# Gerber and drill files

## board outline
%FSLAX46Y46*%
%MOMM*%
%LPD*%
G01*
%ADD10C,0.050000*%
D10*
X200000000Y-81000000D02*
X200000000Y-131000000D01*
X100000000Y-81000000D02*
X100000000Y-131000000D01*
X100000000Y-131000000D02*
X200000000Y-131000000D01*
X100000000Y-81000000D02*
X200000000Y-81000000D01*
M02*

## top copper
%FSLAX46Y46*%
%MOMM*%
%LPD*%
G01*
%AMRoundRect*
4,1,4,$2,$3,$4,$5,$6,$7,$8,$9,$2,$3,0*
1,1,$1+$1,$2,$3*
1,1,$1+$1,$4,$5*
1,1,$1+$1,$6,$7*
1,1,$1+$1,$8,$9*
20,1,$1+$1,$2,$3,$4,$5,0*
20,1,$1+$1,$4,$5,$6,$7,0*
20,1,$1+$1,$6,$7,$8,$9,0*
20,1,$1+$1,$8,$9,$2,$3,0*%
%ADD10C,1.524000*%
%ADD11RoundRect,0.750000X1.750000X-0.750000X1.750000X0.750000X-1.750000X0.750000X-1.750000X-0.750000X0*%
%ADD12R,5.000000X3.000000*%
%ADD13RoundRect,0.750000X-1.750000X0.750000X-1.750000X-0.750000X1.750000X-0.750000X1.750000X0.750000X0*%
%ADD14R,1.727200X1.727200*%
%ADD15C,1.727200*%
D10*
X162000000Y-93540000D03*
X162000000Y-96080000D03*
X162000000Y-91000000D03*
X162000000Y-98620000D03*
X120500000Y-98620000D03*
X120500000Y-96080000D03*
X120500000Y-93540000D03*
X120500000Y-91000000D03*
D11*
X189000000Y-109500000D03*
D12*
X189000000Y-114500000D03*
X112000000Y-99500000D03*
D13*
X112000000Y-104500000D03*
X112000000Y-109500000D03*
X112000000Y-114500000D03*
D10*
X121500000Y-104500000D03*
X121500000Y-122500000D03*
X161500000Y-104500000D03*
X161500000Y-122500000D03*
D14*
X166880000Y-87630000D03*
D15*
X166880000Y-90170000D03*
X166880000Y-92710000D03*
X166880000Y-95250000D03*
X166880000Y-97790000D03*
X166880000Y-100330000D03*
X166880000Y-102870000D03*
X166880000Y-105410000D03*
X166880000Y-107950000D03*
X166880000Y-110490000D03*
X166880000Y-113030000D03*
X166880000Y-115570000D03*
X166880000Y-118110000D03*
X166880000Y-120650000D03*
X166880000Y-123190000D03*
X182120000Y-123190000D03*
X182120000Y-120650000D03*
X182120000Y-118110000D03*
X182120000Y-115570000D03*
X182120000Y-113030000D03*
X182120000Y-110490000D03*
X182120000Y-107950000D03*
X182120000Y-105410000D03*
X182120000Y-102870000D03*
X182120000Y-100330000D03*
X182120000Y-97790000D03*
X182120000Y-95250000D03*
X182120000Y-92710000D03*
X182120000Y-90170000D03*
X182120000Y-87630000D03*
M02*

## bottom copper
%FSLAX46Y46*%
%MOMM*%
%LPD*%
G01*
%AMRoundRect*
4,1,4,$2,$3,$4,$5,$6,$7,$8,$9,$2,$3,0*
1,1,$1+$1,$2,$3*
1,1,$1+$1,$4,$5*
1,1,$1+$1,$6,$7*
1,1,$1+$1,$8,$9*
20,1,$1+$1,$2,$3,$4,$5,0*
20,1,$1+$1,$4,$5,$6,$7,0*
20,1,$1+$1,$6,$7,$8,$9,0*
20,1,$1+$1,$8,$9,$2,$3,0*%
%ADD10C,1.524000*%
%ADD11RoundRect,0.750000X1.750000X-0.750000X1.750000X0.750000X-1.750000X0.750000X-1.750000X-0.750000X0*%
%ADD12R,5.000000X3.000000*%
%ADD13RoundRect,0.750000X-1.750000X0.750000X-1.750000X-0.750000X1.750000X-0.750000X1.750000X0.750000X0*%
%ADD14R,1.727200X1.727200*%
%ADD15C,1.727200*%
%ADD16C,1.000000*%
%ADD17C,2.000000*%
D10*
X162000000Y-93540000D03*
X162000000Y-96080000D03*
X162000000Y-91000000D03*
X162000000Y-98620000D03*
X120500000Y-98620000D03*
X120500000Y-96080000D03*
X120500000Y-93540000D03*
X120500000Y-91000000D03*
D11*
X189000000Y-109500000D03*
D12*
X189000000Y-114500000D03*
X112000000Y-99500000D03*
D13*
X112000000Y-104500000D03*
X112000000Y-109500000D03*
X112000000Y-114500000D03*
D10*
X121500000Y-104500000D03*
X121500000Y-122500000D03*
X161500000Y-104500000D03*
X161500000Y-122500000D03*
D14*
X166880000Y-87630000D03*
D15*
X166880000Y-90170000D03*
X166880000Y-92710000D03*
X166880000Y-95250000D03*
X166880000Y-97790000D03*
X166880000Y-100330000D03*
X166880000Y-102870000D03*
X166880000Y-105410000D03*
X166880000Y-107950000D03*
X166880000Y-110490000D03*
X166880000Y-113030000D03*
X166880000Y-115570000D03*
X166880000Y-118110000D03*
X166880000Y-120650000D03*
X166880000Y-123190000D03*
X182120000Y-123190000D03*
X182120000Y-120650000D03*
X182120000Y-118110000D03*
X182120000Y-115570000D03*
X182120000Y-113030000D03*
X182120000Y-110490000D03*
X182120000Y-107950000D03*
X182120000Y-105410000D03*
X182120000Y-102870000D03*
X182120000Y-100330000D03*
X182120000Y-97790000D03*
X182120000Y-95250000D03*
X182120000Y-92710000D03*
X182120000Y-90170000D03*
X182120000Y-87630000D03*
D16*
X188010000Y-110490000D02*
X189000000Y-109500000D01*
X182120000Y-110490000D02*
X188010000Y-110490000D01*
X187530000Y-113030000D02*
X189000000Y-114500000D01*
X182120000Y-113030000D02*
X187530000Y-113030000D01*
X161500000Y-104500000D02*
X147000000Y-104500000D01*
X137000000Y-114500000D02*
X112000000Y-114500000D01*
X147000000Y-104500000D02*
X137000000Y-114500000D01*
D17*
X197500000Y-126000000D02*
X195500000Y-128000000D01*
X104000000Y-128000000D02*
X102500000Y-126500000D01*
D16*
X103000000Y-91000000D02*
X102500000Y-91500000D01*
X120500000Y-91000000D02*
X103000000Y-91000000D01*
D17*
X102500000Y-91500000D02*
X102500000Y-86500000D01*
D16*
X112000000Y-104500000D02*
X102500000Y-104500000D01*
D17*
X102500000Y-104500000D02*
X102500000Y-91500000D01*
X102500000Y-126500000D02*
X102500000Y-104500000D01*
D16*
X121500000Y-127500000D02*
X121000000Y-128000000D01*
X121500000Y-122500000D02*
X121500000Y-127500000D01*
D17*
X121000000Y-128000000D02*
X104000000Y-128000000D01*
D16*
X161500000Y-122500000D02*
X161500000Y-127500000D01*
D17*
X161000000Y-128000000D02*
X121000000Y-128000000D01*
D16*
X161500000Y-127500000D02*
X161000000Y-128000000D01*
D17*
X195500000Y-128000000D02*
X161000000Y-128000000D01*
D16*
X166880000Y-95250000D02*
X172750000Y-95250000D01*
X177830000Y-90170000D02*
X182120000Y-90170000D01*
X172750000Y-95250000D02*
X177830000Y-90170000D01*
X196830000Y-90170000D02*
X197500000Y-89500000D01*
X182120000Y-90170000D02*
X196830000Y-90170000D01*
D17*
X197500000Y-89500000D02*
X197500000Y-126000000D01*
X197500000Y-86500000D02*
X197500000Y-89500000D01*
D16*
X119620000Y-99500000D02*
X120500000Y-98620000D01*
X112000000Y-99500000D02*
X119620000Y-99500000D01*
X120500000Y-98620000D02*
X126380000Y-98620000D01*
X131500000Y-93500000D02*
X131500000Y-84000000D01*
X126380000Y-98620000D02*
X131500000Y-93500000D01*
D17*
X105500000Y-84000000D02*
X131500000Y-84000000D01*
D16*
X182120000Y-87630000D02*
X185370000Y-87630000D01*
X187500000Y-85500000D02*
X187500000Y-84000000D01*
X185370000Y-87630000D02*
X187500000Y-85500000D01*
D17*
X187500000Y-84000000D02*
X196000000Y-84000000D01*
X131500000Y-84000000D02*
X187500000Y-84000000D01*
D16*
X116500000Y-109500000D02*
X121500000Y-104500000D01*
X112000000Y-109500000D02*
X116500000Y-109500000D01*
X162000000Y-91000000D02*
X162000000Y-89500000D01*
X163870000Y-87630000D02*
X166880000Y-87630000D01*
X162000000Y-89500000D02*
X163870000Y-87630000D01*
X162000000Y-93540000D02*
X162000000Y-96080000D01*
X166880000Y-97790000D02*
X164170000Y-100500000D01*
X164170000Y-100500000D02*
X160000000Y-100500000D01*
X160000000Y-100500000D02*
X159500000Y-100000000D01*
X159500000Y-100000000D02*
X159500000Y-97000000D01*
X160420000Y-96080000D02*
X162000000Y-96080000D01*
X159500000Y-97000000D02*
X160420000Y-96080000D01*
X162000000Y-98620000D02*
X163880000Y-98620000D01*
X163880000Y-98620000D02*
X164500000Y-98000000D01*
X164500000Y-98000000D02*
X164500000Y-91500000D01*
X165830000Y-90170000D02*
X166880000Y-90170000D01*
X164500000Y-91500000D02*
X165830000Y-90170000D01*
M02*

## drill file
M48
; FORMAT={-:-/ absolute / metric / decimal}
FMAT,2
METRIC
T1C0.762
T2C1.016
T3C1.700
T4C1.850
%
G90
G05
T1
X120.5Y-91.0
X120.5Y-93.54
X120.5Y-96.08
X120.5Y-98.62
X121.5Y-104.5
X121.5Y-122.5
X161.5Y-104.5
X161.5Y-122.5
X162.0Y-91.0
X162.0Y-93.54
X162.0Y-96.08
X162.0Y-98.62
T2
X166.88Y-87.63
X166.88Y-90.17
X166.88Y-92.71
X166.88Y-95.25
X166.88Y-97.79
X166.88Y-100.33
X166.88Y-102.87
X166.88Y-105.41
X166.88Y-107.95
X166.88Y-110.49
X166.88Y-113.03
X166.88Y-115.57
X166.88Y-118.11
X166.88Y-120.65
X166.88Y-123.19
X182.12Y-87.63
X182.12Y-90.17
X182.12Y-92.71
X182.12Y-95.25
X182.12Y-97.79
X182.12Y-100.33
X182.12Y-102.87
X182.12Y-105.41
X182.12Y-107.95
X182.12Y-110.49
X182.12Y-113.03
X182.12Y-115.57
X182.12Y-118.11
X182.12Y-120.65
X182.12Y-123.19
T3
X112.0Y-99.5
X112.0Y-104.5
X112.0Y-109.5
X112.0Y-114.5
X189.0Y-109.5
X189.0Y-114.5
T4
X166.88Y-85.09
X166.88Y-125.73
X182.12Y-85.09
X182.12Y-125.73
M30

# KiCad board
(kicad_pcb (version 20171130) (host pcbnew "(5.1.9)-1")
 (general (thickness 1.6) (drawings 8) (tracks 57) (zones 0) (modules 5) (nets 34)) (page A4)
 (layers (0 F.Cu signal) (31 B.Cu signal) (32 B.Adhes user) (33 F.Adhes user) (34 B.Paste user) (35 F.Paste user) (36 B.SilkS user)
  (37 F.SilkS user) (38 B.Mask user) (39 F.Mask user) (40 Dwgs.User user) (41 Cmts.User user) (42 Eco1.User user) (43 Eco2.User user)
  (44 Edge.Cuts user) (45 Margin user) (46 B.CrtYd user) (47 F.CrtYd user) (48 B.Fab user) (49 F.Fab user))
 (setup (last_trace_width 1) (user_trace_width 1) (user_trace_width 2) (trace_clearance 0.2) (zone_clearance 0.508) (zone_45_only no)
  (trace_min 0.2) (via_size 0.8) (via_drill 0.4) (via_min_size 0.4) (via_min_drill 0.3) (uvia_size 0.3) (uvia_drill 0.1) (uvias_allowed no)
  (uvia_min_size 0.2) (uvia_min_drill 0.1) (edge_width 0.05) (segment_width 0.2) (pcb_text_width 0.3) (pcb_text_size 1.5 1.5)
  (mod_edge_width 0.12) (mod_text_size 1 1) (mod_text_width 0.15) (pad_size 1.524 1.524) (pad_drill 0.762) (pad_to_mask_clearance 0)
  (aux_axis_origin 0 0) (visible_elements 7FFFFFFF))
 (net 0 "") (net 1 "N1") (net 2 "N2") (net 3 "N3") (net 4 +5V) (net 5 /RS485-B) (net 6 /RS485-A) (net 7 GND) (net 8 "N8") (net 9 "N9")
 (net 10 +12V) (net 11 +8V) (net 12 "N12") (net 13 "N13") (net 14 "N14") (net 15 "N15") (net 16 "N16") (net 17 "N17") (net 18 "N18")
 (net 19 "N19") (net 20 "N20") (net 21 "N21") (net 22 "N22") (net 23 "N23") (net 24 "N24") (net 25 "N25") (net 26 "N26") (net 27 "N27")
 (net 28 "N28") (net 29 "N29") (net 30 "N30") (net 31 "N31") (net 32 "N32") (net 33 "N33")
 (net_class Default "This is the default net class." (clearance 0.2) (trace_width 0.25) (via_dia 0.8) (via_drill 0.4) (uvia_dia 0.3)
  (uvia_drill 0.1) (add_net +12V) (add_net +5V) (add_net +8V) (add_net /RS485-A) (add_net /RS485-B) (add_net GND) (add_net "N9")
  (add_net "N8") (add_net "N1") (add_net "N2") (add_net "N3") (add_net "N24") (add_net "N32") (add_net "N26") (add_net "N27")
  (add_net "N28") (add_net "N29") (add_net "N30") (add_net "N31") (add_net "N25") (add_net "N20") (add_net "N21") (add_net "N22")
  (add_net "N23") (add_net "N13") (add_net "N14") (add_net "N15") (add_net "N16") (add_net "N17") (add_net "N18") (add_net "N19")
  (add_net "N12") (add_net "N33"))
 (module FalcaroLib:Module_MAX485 (layer F.Cu) (at 120.5 91)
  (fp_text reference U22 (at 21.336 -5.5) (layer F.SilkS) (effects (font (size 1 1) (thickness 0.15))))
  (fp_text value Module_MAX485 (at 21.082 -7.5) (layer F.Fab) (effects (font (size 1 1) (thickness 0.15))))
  (pad DE thru_hole circle (at 41.5 2.54) (size 1.524 1.524) (drill 0.762) (layers *.Cu *.Mask) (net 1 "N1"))
  (pad RE thru_hole circle (at 41.5 5.08) (size 1.524 1.524) (drill 0.762) (layers *.Cu *.Mask) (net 1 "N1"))
  (pad DI thru_hole circle (at 41.5 0) (size 1.524 1.524) (drill 0.762) (layers *.Cu *.Mask) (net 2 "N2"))
  (pad RO thru_hole circle (at 41.5 7.62) (size 1.524 1.524) (drill 0.762) (layers *.Cu *.Mask) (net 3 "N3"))
  (pad VCC thru_hole circle (at 0 7.62) (size 1.524 1.524) (drill 0.762) (layers *.Cu *.Mask) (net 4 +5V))
  (pad B thru_hole circle (at 0 5.08) (size 1.524 1.524) (drill 0.762) (layers *.Cu *.Mask) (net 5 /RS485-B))
  (pad A thru_hole circle (at 0 2.54) (size 1.524 1.524) (drill 0.762) (layers *.Cu *.Mask) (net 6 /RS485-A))
  (pad GND thru_hole circle (at 0 0) (size 1.524 1.524) (drill 0.762) (layers *.Cu *.Mask) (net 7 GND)))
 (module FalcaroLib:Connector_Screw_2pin (layer F.Cu) (at 184.5 118 90)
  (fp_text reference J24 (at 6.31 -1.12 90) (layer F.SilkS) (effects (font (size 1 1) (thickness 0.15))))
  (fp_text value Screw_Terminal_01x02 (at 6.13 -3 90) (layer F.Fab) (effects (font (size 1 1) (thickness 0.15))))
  (pad 2 thru_hole roundrect (at 8.5 4.5 90) (size 3 5) (drill 1.7) (layers *.Cu *.Mask) (roundrect_rratio 0.25) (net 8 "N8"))
  (pad 1 thru_hole rect (at 3.5 4.5 90) (size 3 5) (drill 1.7) (layers *.Cu *.Mask) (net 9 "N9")))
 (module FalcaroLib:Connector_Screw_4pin (layer F.Cu) (at 116.5 96 270)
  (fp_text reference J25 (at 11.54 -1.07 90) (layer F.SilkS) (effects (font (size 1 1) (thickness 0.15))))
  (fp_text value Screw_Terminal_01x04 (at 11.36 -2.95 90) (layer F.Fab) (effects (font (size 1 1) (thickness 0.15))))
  (pad 1 thru_hole rect (at 3.5 4.5 270) (size 3 5) (drill 1.7) (layers *.Cu *.Mask) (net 4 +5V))
  (pad 2 thru_hole roundrect (at 8.5 4.5 270) (size 3 5) (drill 1.7) (layers *.Cu *.Mask) (roundrect_rratio 0.25) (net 7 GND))
  (pad 3 thru_hole roundrect (at 13.5 4.5 270) (size 3 5) (drill 1.7) (layers *.Cu *.Mask) (roundrect_rratio 0.25) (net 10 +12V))
  (pad 4 thru_hole roundrect (at 18.5 4.5 270) (size 3 5) (drill 1.7) (layers *.Cu *.Mask) (roundrect_rratio 0.25) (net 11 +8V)))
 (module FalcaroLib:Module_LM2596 (layer F.Cu) (at 121.5 104.5)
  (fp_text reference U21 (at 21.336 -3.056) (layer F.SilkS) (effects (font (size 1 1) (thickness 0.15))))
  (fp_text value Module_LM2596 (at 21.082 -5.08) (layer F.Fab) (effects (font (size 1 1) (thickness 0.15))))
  (pad IN+ thru_hole circle (at 0 0) (size 1.524 1.524) (drill 0.762) (layers *.Cu *.Mask) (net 10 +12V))
  (pad IN- thru_hole circle (at 0 18) (size 1.524 1.524) (drill 0.762) (layers *.Cu *.Mask) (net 7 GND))
  (pad OUT+ thru_hole circle (at 40 0) (size 1.524 1.524) (drill 0.762) (layers *.Cu *.Mask) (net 11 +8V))
  (pad OUT- thru_hole circle (at 40 18) (size 1.524 1.524) (drill 0.762) (layers *.Cu *.Mask) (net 7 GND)))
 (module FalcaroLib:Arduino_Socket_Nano (layer F.Cu) (at 174.5 127)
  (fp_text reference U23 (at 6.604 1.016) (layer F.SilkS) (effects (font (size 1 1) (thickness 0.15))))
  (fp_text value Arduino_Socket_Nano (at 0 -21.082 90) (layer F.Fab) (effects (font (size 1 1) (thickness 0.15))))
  (pad "" np_thru_hole circle (at 7.62 -1.27) (size 1.85 1.85) (drill 1.85) (layers *.Cu *.Mask))
  (pad "" np_thru_hole circle (at -7.62 -1.27) (size 1.85 1.85) (drill 1.85) (layers *.Cu *.Mask))
  (pad "" np_thru_hole circle (at 7.62 -41.91) (size 1.85 1.85) (drill 1.85) (layers *.Cu *.Mask))
  (pad "" np_thru_hole circle (at -7.62 -41.91) (size 1.85 1.85) (drill 1.85) (layers *.Cu *.Mask))
  (pad D1 thru_hole rect (at -7.62 -39.37) (size 1.7272 1.7272) (drill 1.016) (layers *.Cu *.Mask) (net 2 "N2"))
  (pad D0 thru_hole circle (at -7.62 -36.83) (size 1.7272 1.7272) (drill 1.016) (layers *.Cu *.Mask) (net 3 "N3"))
  (pad RST1 thru_hole circle (at -7.62 -34.29) (size 1.7272 1.7272) (drill 1.016) (layers *.Cu *.Mask) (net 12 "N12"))
  (pad GND1 thru_hole circle (at -7.62 -31.75) (size 1.7272 1.7272) (drill 1.016) (layers *.Cu *.Mask) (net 7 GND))
  (pad D2 thru_hole circle (at -7.62 -29.21) (size 1.7272 1.7272) (drill 1.016) (layers *.Cu *.Mask) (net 1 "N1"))
  (pad D3 thru_hole circle (at -7.62 -26.67) (size 1.7272 1.7272) (drill 1.016) (layers *.Cu *.Mask) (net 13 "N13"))
  (pad D4 thru_hole circle (at -7.62 -24.13) (size 1.7272 1.7272) (drill 1.016) (layers *.Cu *.Mask) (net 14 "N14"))
  (pad D5 thru_hole circle (at -7.62 -21.59) (size 1.7272 1.7272) (drill 1.016) (layers *.Cu *.Mask) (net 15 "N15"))
  (pad D6 thru_hole circle (at -7.62 -19.05) (size 1.7272 1.7272) (drill 1.016) (layers *.Cu *.Mask) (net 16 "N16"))
  (pad D7 thru_hole circle (at -7.62 -16.51) (size 1.7272 1.7272) (drill 1.016) (layers *.Cu *.Mask) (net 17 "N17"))
  (pad D8 thru_hole circle (at -7.62 -13.97) (size 1.7272 1.7272) (drill 1.016) (layers *.Cu *.Mask) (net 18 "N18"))
  (pad D9 thru_hole circle (at -7.62 -11.43) (size 1.7272 1.7272) (drill 1.016) (layers *.Cu *.Mask) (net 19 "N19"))
  (pad D10 thru_hole circle (at -7.62 -8.89) (size 1.7272 1.7272) (drill 1.016) (layers *.Cu *.Mask) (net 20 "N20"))
  (pad D11 thru_hole circle (at -7.62 -6.35) (size 1.7272 1.7272) (drill 1.016) (layers *.Cu *.Mask) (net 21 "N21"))
  (pad D12 thru_hole circle (at -7.62 -3.81) (size 1.7272 1.7272) (drill 1.016) (layers *.Cu *.Mask) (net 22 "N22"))
  (pad D13 thru_hole circle (at 7.62 -3.81) (size 1.7272 1.7272) (drill 1.016) (layers *.Cu *.Mask) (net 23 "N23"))
  (pad 3V3 thru_hole circle (at 7.62 -6.35) (size 1.7272 1.7272) (drill 1.016) (layers *.Cu *.Mask) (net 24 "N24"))
  (pad AREF thru_hole circle (at 7.62 -8.89) (size 1.7272 1.7272) (drill 1.016) (layers *.Cu *.Mask) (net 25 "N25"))
  (pad A0 thru_hole circle (at 7.62 -11.43) (size 1.7272 1.7272) (drill 1.016) (layers *.Cu *.Mask) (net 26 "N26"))
  (pad A1 thru_hole circle (at 7.62 -13.97) (size 1.7272 1.7272) (drill 1.016) (layers *.Cu *.Mask) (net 9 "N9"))
  (pad A2 thru_hole circle (at 7.62 -16.51) (size 1.7272 1.7272) (drill 1.016) (layers *.Cu *.Mask) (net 8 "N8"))
  (pad A3 thru_hole circle (at 7.62 -19.05) (size 1.7272 1.7272) (drill 1.016) (layers *.Cu *.Mask) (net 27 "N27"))
  (pad A4 thru_hole circle (at 7.62 -21.59) (size 1.7272 1.7272) (drill 1.016) (layers *.Cu *.Mask) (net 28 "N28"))
  (pad A5 thru_hole circle (at 7.62 -24.13) (size 1.7272 1.7272) (drill 1.016) (layers *.Cu *.Mask) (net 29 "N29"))
  (pad A6 thru_hole circle (at 7.62 -26.67) (size 1.7272 1.7272) (drill 1.016) (layers *.Cu *.Mask) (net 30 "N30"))
  (pad A7 thru_hole circle (at 7.62 -29.21) (size 1.7272 1.7272) (drill 1.016) (layers *.Cu *.Mask) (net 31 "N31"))
  (pad 5V thru_hole circle (at 7.62 -31.75) (size 1.7272 1.7272) (drill 1.016) (layers *.Cu *.Mask) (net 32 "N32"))
  (pad RST2 thru_hole circle (at 7.62 -34.29) (size 1.7272 1.7272) (drill 1.016) (layers *.Cu *.Mask) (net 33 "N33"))
  (pad GND2 thru_hole circle (at 7.62 -36.83) (size 1.7272 1.7272) (drill 1.016) (layers *.Cu *.Mask) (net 7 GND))
  (pad VIN thru_hole circle (at 7.62 -39.37) (size 1.7272 1.7272) (drill 1.016) (layers *.Cu *.Mask) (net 4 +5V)))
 (gr_line (start 200 81) (end 200 131) (layer Edge.Cuts) (width 0.05))
 (gr_line (start 100 81) (end 100 131) (layer Edge.Cuts) (width 0.05))
 (gr_line (start 100 131) (end 200 131) (layer Edge.Cuts) (width 0.05))
 (gr_line (start 100 81) (end 200 81) (layer Edge.Cuts) (width 0.05))
 (segment (start 188.01 110.49) (end 189 109.5) (width 1) (layer B.Cu) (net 8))
 (segment (start 182.12 110.49) (end 188.01 110.49) (width 1) (layer B.Cu) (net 8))
 (segment (start 187.53 113.03) (end 189 114.5) (width 1) (layer B.Cu) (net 9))
 (segment (start 182.12 113.03) (end 187.53 113.03) (width 1) (layer B.Cu) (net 9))
 (segment (start 161.5 104.5) (end 147 104.5) (width 1) (layer B.Cu) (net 11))
 (segment (start 137 114.5) (end 112 114.5) (width 1) (layer B.Cu) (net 11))
 (segment (start 147 104.5) (end 137 114.5) (width 1) (layer B.Cu) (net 11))
 (segment (start 197.5 126) (end 195.5 128) (width 2) (layer B.Cu) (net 7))
 (segment (start 104 128) (end 102.5 126.5) (width 2) (layer B.Cu) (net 7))
 (segment (start 103 91) (end 102.5 91.5) (width 1) (layer B.Cu) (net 7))
 (segment (start 120.5 91) (end 103 91) (width 1) (layer B.Cu) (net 7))
 (segment (start 102.5 91.5) (end 102.5 86.5) (width 2) (layer B.Cu) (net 7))
 (segment (start 112 104.5) (end 102.5 104.5) (width 1) (layer B.Cu) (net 7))
 (segment (start 102.5 104.5) (end 102.5 91.5) (width 2) (layer B.Cu) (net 7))
 (segment (start 102.5 126.5) (end 102.5 104.5) (width 2) (layer B.Cu) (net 7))
 (segment (start 121.5 127.5) (end 121 128) (width 1) (layer B.Cu) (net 7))
 (segment (start 121.5 122.5) (end 121.5 127.5) (width 1) (layer B.Cu) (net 7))
 (segment (start 121 128) (end 104 128) (width 2) (layer B.Cu) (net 7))
 (segment (start 161.5 122.5) (end 161.5 127.5) (width 1) (layer B.Cu) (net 7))
 (segment (start 161 128) (end 121 128) (width 2) (layer B.Cu) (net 7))
 (segment (start 161.5 127.5) (end 161 128) (width 1) (layer B.Cu) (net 7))
 (segment (start 195.5 128) (end 161 128) (width 2) (layer B.Cu) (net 7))
 (segment (start 166.88 95.25) (end 172.75 95.25) (width 1) (layer B.Cu) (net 7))
 (segment (start 177.83 90.17) (end 182.12 90.17) (width 1) (layer B.Cu) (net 7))
 (segment (start 172.75 95.25) (end 177.83 90.17) (width 1) (layer B.Cu) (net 7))
 (segment (start 196.83 90.17) (end 197.5 89.5) (width 1) (layer B.Cu) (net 7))
 (segment (start 182.12 90.17) (end 196.83 90.17) (width 1) (layer B.Cu) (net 7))
 (segment (start 197.5 89.5) (end 197.5 126) (width 2) (layer B.Cu) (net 7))
 (segment (start 197.5 86.5) (end 197.5 89.5) (width 2) (layer B.Cu) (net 7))
 (segment (start 119.62 99.5) (end 120.5 98.62) (width 1) (layer B.Cu) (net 4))
 (segment (start 112 99.5) (end 119.62 99.5) (width 1) (layer B.Cu) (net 4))
 (segment (start 120.5 98.62) (end 126.38 98.62) (width 1) (layer B.Cu) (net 4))
 (segment (start 131.5 93.5) (end 131.5 84) (width 1) (layer B.Cu) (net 4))
 (segment (start 126.38 98.62) (end 131.5 93.5) (width 1) (layer B.Cu) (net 4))
 (segment (start 105.5 84) (end 131.5 84) (width 2) (layer B.Cu) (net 4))
 (segment (start 182.12 87.63) (end 185.37 87.63) (width 1) (layer B.Cu) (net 4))
 (segment (start 187.5 85.5) (end 187.5 84) (width 1) (layer B.Cu) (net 4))
 (segment (start 185.37 87.63) (end 187.5 85.5) (width 1) (layer B.Cu) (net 4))
 (segment (start 187.5 84) (end 196 84) (width 2) (layer B.Cu) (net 4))
 (segment (start 131.5 84) (end 187.5 84) (width 2) (layer B.Cu) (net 4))
 (segment (start 116.5 109.5) (end 121.5 104.5) (width 1) (layer B.Cu) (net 10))
 (segment (start 112 109.5) (end 116.5 109.5) (width 1) (layer B.Cu) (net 10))
 (segment (start 162 91) (end 162 89.5) (width 1) (layer B.Cu) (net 2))
 (segment (start 163.87 87.63) (end 166.88 87.63) (width 1) (layer B.Cu) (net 2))
 (segment (start 162 89.5) (end 163.87 87.63) (width 1) (layer B.Cu) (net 2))
 (segment (start 162 93.54) (end 162 96.08) (width 1) (layer B.Cu) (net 1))
 (segment (start 166.88 97.79) (end 164.17 100.5) (width 1) (layer B.Cu) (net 1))
 (segment (start 164.17 100.5) (end 160 100.5) (width 1) (layer B.Cu) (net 1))
 (segment (start 160 100.5) (end 159.5 100) (width 1) (layer B.Cu) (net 1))
 (segment (start 159.5 100) (end 159.5 97) (width 1) (layer B.Cu) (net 1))
 (segment (start 160.42 96.08) (end 162 96.08) (width 1) (layer B.Cu) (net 1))
 (segment (start 159.5 97) (end 160.42 96.08) (width 1) (layer B.Cu) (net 1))
 (segment (start 162 98.62) (end 163.88 98.62) (width 1) (layer B.Cu) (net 3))
 (segment (start 163.88 98.62) (end 164.5 98) (width 1) (layer B.Cu) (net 3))
 (segment (start 164.5 98) (end 164.5 91.5) (width 1) (layer B.Cu) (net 3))
 (segment (start 165.83 90.17) (end 166.88 90.17) (width 1) (layer B.Cu) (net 3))
 (segment (start 164.5 91.5) (end 165.83 90.17) (width 1) (layer B.Cu) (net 3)))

